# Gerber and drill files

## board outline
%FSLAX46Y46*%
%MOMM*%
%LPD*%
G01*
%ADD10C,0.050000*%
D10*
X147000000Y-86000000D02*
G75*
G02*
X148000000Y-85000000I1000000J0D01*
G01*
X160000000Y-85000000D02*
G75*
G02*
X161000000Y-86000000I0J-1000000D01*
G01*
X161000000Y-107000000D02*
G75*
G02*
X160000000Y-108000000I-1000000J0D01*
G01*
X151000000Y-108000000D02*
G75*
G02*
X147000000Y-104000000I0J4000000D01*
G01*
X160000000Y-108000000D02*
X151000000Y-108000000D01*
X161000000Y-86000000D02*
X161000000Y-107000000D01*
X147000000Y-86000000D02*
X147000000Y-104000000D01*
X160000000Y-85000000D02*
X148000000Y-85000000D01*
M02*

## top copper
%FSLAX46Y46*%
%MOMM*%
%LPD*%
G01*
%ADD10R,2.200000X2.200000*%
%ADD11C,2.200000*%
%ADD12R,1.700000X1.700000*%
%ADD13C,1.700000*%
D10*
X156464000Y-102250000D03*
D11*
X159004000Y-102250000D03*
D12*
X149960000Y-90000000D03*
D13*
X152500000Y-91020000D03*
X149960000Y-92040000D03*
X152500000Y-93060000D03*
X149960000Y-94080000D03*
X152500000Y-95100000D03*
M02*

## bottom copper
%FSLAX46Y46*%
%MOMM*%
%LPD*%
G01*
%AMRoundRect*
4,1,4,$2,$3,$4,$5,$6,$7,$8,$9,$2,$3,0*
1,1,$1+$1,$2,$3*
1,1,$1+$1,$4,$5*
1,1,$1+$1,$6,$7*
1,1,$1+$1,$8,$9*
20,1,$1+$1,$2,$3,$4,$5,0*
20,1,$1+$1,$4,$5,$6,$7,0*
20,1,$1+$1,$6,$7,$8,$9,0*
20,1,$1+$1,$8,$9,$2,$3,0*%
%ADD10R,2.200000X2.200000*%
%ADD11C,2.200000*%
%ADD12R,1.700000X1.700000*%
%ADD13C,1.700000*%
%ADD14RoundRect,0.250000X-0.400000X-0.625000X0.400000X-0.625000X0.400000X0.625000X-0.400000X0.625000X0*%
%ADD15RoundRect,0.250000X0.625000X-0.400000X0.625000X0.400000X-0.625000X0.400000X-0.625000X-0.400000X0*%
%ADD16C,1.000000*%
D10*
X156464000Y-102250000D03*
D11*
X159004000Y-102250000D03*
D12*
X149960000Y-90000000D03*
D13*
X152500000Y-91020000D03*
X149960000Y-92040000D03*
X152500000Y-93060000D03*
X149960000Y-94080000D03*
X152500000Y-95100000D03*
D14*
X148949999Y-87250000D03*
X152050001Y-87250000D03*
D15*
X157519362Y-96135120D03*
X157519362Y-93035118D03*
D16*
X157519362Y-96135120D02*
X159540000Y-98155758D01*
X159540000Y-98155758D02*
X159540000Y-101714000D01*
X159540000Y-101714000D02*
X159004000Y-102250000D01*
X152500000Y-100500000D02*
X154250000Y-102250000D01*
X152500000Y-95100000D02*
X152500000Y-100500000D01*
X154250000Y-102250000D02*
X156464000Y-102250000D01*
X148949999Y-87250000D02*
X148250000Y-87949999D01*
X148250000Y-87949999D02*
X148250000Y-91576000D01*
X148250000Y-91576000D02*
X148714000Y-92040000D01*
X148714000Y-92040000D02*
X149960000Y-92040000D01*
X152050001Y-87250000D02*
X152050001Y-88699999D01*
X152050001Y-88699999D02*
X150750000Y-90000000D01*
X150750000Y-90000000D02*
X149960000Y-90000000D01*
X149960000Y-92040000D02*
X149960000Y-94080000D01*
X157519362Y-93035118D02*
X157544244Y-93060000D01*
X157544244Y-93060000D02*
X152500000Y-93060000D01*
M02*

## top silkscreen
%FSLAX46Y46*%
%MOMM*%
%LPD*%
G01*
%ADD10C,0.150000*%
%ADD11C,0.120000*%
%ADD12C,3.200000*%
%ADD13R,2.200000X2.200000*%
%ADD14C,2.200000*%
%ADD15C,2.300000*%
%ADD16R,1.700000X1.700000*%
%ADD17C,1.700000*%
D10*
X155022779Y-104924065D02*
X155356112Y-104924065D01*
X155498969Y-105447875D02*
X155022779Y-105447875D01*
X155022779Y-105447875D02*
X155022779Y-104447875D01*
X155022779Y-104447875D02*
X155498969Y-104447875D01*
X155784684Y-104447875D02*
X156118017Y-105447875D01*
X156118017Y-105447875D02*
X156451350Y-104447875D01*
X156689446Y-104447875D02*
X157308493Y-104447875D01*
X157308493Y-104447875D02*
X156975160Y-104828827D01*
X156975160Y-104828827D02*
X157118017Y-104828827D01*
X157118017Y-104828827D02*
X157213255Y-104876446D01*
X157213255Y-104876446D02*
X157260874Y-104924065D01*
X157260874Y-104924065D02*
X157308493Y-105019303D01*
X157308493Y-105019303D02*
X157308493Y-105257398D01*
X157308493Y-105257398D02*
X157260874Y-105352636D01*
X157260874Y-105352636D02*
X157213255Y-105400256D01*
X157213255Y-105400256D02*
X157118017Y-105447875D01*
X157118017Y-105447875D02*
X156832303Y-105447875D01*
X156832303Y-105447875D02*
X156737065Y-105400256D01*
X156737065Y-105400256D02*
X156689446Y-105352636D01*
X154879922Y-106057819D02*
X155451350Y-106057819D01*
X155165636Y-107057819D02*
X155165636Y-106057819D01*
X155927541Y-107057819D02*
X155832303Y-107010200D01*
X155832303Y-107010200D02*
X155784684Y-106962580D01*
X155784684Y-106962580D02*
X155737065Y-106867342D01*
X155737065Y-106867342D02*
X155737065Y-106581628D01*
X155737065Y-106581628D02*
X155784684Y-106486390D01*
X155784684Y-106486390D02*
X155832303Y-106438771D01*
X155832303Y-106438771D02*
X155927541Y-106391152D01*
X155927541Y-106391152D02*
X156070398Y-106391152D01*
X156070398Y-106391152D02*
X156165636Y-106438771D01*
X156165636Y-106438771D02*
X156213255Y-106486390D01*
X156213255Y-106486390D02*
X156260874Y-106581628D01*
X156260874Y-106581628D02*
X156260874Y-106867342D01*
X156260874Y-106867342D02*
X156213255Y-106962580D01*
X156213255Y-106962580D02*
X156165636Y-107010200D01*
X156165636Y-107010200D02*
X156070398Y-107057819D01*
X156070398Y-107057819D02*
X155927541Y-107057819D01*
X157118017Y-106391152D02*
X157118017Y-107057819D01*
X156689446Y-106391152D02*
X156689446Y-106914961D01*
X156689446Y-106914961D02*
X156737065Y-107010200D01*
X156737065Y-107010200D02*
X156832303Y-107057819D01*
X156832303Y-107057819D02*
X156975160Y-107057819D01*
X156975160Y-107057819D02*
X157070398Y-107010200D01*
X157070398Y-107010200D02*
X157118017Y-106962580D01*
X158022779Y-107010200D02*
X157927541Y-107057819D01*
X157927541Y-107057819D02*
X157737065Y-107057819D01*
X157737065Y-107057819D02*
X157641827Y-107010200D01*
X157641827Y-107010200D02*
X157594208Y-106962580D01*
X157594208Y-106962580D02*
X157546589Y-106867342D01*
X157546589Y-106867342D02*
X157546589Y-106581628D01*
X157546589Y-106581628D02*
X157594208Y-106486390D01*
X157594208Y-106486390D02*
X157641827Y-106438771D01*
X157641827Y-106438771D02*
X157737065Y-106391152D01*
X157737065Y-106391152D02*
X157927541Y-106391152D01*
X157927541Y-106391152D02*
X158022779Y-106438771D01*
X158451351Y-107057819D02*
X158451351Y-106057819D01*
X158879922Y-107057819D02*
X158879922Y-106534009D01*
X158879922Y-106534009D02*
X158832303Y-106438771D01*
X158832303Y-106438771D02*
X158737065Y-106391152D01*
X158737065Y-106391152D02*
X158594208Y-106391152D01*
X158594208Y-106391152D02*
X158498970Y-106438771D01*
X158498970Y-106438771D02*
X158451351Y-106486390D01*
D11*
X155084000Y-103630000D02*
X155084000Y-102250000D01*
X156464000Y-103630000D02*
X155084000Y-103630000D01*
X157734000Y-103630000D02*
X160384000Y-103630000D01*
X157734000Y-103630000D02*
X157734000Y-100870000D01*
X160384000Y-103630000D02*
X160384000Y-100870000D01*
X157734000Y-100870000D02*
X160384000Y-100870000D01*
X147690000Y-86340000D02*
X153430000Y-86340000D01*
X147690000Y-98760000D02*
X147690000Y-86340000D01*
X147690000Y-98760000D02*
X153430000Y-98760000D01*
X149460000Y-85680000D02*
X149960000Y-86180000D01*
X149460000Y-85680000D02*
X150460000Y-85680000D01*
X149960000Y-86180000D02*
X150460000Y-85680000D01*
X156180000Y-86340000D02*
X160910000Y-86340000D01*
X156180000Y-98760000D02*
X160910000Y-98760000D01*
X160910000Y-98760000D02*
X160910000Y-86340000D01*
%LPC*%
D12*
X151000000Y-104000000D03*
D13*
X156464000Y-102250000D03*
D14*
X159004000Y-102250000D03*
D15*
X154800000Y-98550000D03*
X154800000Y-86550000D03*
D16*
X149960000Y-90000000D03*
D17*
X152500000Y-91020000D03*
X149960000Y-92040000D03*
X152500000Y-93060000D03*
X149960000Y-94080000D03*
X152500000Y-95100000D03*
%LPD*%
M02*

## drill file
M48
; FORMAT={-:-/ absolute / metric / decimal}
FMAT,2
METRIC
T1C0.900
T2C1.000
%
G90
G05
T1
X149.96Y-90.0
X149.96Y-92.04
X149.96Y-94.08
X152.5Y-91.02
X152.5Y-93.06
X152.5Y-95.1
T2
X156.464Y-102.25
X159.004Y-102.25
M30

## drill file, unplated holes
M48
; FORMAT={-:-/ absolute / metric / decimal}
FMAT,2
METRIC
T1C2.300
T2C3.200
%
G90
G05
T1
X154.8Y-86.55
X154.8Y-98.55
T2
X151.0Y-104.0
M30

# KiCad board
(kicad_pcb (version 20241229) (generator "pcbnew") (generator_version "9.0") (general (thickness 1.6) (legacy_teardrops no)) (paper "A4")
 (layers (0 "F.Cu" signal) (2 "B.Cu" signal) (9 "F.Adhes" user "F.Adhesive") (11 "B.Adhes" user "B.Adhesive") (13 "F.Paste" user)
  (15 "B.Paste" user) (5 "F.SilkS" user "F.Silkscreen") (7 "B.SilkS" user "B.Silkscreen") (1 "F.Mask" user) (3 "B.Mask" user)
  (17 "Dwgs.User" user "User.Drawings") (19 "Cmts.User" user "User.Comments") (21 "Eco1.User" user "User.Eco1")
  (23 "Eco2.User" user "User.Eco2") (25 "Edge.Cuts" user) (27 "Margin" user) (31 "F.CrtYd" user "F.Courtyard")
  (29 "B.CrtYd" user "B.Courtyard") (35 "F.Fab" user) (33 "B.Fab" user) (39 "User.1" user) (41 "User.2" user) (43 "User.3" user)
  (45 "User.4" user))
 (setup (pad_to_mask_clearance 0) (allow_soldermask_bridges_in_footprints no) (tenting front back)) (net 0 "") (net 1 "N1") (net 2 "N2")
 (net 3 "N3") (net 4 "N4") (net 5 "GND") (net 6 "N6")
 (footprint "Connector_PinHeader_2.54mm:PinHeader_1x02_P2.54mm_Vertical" (layer "F.Cu") (at 156.464 102.25 90)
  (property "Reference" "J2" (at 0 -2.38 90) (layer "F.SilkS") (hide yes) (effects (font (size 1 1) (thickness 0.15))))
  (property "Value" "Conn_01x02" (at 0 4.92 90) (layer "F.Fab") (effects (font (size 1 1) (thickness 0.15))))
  (fp_line (start -1.38 -1.38) (end 0 -1.38) (stroke (width 0.12) (type solid)) (layer "F.SilkS"))
  (fp_line (start -1.38 0) (end -1.38 -1.38) (stroke (width 0.12) (type solid)) (layer "F.SilkS"))
  (fp_line (start 1.38 1.27) (end 1.38 3.92) (stroke (width 0.12) (type solid)) (layer "F.SilkS"))
  (fp_line (start -1.38 1.27) (end 1.38 1.27) (stroke (width 0.12) (type solid)) (layer "F.SilkS"))
  (fp_line (start -1.38 1.27) (end -1.38 3.92) (stroke (width 0.12) (type solid)) (layer "F.SilkS"))
  (fp_line (start -1.38 3.92) (end 1.38 3.92) (stroke (width 0.12) (type solid)) (layer "F.SilkS"))
  (pad "1" thru_hole rect (at 0 0 90) (size 2.2 2.2) (drill 1) (layers "*.Cu" "*.Mask") (remove_unused_layers no) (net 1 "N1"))
  (pad "2" thru_hole circle (at 0 2.54 90) (size 2.2 2.2) (drill 1) (layers "*.Cu" "*.Mask") (remove_unused_layers no) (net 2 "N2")))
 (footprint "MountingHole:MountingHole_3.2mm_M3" (layer "F.Cu") (at 151 104)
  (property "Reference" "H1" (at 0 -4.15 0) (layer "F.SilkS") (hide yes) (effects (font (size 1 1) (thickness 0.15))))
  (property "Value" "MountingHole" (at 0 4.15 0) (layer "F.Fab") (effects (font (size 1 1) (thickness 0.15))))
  (pad "" np_thru_hole circle (at 0 0) (size 3.2 3.2) (drill 3.2) (layers "*.Cu" "*.Mask")))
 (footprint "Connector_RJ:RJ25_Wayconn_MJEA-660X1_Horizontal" (layer "F.Cu") (at 149.96 90 90)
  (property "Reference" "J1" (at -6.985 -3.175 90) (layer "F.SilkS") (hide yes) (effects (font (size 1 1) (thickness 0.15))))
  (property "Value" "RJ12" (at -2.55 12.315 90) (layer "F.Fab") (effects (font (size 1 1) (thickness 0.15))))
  (fp_line (start 3.66 -2.27) (end 3.66 3.47) (stroke (width 0.12) (type solid)) (layer "F.SilkS"))
  (fp_line (start -8.76 -2.27) (end 3.66 -2.27) (stroke (width 0.12) (type solid)) (layer "F.SilkS"))
  (fp_line (start -8.76 -2.27) (end -8.76 3.47) (stroke (width 0.12) (type solid)) (layer "F.SilkS"))
  (fp_line (start 4.32 -0.5) (end 3.82 0) (stroke (width 0.12) (type solid)) (layer "F.SilkS"))
  (fp_line (start 4.32 -0.5) (end 4.32 0.5) (stroke (width 0.12) (type solid)) (layer "F.SilkS"))
  (fp_line (start 3.82 0) (end 4.32 0.5) (stroke (width 0.12) (type solid)) (layer "F.SilkS"))
  (fp_line (start 3.66 6.22) (end 3.66 10.95) (stroke (width 0.12) (type solid)) (layer "F.SilkS"))
  (fp_line (start -8.76 6.22) (end -8.76 10.95) (stroke (width 0.12) (type solid)) (layer "F.SilkS"))
  (fp_line (start -8.76 10.95) (end 3.66 10.95) (stroke (width 0.12) (type solid)) (layer "F.SilkS"))
  (pad "" np_thru_hole circle (at -8.55 4.84 90) (size 2.3 2.3) (drill 2.3) (layers "*.Cu" "*.Mask"))
  (pad "" np_thru_hole circle (at 3.45 4.84 90) (size 2.3 2.3) (drill 2.3) (layers "*.Cu" "*.Mask"))
  (pad "1" thru_hole rect (at 0 0 90) (size 1.7 1.7) (drill 0.9) (layers "*.Cu" "*.Mask") (remove_unused_layers no) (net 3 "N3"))
  (pad "2" thru_hole circle (at -1.02 2.54 90) (size 1.7 1.7) (drill 0.9) (layers "*.Cu" "*.Mask") (remove_unused_layers no) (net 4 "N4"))
  (pad "3" thru_hole circle (at -2.04 0 90) (size 1.7 1.7) (drill 0.9) (layers "*.Cu" "*.Mask") (remove_unused_layers no) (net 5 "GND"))
  (pad "4" thru_hole circle (at -3.06 2.54 90) (size 1.7 1.7) (drill 0.9) (layers "*.Cu" "*.Mask") (remove_unused_layers no) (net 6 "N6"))
  (pad "5" thru_hole circle (at -4.08 0 90) (size 1.7 1.7) (drill 0.9) (layers "*.Cu" "*.Mask") (remove_unused_layers no) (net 5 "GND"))
  (pad "6" thru_hole circle (at -5.1 2.54 90) (size 1.7 1.7) (drill 0.9) (layers "*.Cu" "*.Mask") (remove_unused_layers no) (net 1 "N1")))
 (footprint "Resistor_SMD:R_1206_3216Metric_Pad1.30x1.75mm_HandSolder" (layer "B.Cu") (at 150.5 87.25)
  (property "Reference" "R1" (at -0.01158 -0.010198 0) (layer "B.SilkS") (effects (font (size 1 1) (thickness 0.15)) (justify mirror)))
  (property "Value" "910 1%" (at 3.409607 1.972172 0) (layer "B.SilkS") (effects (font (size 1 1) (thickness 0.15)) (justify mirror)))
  (pad "1" smd roundrect (at -1.550001 0) (size 1.3 1.75) (layers "B.Cu" "B.Mask" "B.Paste") (roundrect_rratio 0.192308) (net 5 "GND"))
  (pad "2" smd roundrect (at 1.550001 0) (size 1.3 1.75) (layers "B.Cu" "B.Mask" "B.Paste") (roundrect_rratio 0.192308) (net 3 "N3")))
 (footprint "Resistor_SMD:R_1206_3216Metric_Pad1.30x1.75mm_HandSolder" (layer "B.Cu") (at 157.519362 94.585119 90)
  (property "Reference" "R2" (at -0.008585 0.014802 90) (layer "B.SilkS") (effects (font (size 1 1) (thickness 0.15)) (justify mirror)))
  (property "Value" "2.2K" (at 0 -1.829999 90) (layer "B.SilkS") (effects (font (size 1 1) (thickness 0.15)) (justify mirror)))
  (pad "1" smd roundrect (at -1.550001 0 90) (size 1.3 1.75) (layers "B.Cu" "B.Mask" "B.Paste") (roundrect_rratio 0.192308) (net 2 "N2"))
  (pad "2" smd roundrect (at 1.550001 0 90) (size 1.3 1.75) (layers "B.Cu" "B.Mask" "B.Paste") (roundrect_rratio 0.192308) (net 6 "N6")))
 (gr_arc (start 147 86) (mid 147.292893 85.292893) (end 148 85) (stroke (width 0.05) (type default)) (layer "Edge.Cuts"))
 (gr_line (start 160 85) (end 148 85) (stroke (width 0.05) (type default)) (layer "Edge.Cuts"))
 (gr_line (start 161 86) (end 161 107) (stroke (width 0.05) (type default)) (layer "Edge.Cuts"))
 (gr_line (start 160 108) (end 151 108) (stroke (width 0.05) (type default)) (layer "Edge.Cuts"))
 (gr_arc (start 161 107) (mid 160.707107 107.707107) (end 160 108) (stroke (width 0.05) (type default)) (layer "Edge.Cuts"))
 (gr_arc (start 160 85) (mid 160.707107 85.292893) (end 161 86) (stroke (width 0.05) (type default)) (layer "Edge.Cuts"))
 (gr_arc (start 151 108) (mid 148.171573 106.828427) (end 147 104) (stroke (width 0.05) (type default)) (layer "Edge.Cuts"))
 (gr_line (start 147 86) (end 147 104) (stroke (width 0.05) (type default)) (layer "Edge.Cuts"))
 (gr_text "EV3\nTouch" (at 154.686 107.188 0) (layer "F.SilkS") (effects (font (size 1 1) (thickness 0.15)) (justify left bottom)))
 (segment (start 149.96 92.04) (end 149.96 94.08) (width 1) (layer "B.Cu") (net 5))
 (segment (start 148.714 92.04) (end 149.96 92.04) (width 1) (layer "B.Cu") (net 5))
 (segment (start 148.25 87.949999) (end 148.25 91.576) (width 1) (layer "B.Cu") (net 5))
 (segment (start 148.25 91.576) (end 148.714 92.04) (width 1) (layer "B.Cu") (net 5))
 (segment (start 148.949999 87.25) (end 148.25 87.949999) (width 1) (layer "B.Cu") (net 5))
 (segment (start 152.050001 87.25) (end 152.050001 88.699999) (width 1) (layer "B.Cu") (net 3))
 (segment (start 152.050001 88.699999) (end 150.75 90) (width 1) (layer "B.Cu") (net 3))
 (segment (start 150.75 90) (end 149.96 90) (width 1) (layer "B.Cu") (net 3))
 (segment (start 157.519362 93.035118) (end 157.544244 93.06) (width 1) (layer "B.Cu") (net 6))
 (segment (start 157.544244 93.06) (end 152.5 93.06) (width 1) (layer "B.Cu") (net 6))
 (segment (start 152.5 100.5) (end 154.25 102.25) (width 1) (layer "B.Cu") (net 1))
 (segment (start 154.25 102.25) (end 156.464 102.25) (width 1) (layer "B.Cu") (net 1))
 (segment (start 152.5 95.1) (end 152.5 100.5) (width 1) (layer "B.Cu") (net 1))
 (segment (start 157.519362 96.13512) (end 159.54 98.155758) (width 1) (layer "B.Cu") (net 2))
 (segment (start 159.54 101.714) (end 159.004 102.25) (width 1) (layer "B.Cu") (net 2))
 (segment (start 159.54 98.155758) (end 159.54 101.714) (width 1) (layer "B.Cu") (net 2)))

